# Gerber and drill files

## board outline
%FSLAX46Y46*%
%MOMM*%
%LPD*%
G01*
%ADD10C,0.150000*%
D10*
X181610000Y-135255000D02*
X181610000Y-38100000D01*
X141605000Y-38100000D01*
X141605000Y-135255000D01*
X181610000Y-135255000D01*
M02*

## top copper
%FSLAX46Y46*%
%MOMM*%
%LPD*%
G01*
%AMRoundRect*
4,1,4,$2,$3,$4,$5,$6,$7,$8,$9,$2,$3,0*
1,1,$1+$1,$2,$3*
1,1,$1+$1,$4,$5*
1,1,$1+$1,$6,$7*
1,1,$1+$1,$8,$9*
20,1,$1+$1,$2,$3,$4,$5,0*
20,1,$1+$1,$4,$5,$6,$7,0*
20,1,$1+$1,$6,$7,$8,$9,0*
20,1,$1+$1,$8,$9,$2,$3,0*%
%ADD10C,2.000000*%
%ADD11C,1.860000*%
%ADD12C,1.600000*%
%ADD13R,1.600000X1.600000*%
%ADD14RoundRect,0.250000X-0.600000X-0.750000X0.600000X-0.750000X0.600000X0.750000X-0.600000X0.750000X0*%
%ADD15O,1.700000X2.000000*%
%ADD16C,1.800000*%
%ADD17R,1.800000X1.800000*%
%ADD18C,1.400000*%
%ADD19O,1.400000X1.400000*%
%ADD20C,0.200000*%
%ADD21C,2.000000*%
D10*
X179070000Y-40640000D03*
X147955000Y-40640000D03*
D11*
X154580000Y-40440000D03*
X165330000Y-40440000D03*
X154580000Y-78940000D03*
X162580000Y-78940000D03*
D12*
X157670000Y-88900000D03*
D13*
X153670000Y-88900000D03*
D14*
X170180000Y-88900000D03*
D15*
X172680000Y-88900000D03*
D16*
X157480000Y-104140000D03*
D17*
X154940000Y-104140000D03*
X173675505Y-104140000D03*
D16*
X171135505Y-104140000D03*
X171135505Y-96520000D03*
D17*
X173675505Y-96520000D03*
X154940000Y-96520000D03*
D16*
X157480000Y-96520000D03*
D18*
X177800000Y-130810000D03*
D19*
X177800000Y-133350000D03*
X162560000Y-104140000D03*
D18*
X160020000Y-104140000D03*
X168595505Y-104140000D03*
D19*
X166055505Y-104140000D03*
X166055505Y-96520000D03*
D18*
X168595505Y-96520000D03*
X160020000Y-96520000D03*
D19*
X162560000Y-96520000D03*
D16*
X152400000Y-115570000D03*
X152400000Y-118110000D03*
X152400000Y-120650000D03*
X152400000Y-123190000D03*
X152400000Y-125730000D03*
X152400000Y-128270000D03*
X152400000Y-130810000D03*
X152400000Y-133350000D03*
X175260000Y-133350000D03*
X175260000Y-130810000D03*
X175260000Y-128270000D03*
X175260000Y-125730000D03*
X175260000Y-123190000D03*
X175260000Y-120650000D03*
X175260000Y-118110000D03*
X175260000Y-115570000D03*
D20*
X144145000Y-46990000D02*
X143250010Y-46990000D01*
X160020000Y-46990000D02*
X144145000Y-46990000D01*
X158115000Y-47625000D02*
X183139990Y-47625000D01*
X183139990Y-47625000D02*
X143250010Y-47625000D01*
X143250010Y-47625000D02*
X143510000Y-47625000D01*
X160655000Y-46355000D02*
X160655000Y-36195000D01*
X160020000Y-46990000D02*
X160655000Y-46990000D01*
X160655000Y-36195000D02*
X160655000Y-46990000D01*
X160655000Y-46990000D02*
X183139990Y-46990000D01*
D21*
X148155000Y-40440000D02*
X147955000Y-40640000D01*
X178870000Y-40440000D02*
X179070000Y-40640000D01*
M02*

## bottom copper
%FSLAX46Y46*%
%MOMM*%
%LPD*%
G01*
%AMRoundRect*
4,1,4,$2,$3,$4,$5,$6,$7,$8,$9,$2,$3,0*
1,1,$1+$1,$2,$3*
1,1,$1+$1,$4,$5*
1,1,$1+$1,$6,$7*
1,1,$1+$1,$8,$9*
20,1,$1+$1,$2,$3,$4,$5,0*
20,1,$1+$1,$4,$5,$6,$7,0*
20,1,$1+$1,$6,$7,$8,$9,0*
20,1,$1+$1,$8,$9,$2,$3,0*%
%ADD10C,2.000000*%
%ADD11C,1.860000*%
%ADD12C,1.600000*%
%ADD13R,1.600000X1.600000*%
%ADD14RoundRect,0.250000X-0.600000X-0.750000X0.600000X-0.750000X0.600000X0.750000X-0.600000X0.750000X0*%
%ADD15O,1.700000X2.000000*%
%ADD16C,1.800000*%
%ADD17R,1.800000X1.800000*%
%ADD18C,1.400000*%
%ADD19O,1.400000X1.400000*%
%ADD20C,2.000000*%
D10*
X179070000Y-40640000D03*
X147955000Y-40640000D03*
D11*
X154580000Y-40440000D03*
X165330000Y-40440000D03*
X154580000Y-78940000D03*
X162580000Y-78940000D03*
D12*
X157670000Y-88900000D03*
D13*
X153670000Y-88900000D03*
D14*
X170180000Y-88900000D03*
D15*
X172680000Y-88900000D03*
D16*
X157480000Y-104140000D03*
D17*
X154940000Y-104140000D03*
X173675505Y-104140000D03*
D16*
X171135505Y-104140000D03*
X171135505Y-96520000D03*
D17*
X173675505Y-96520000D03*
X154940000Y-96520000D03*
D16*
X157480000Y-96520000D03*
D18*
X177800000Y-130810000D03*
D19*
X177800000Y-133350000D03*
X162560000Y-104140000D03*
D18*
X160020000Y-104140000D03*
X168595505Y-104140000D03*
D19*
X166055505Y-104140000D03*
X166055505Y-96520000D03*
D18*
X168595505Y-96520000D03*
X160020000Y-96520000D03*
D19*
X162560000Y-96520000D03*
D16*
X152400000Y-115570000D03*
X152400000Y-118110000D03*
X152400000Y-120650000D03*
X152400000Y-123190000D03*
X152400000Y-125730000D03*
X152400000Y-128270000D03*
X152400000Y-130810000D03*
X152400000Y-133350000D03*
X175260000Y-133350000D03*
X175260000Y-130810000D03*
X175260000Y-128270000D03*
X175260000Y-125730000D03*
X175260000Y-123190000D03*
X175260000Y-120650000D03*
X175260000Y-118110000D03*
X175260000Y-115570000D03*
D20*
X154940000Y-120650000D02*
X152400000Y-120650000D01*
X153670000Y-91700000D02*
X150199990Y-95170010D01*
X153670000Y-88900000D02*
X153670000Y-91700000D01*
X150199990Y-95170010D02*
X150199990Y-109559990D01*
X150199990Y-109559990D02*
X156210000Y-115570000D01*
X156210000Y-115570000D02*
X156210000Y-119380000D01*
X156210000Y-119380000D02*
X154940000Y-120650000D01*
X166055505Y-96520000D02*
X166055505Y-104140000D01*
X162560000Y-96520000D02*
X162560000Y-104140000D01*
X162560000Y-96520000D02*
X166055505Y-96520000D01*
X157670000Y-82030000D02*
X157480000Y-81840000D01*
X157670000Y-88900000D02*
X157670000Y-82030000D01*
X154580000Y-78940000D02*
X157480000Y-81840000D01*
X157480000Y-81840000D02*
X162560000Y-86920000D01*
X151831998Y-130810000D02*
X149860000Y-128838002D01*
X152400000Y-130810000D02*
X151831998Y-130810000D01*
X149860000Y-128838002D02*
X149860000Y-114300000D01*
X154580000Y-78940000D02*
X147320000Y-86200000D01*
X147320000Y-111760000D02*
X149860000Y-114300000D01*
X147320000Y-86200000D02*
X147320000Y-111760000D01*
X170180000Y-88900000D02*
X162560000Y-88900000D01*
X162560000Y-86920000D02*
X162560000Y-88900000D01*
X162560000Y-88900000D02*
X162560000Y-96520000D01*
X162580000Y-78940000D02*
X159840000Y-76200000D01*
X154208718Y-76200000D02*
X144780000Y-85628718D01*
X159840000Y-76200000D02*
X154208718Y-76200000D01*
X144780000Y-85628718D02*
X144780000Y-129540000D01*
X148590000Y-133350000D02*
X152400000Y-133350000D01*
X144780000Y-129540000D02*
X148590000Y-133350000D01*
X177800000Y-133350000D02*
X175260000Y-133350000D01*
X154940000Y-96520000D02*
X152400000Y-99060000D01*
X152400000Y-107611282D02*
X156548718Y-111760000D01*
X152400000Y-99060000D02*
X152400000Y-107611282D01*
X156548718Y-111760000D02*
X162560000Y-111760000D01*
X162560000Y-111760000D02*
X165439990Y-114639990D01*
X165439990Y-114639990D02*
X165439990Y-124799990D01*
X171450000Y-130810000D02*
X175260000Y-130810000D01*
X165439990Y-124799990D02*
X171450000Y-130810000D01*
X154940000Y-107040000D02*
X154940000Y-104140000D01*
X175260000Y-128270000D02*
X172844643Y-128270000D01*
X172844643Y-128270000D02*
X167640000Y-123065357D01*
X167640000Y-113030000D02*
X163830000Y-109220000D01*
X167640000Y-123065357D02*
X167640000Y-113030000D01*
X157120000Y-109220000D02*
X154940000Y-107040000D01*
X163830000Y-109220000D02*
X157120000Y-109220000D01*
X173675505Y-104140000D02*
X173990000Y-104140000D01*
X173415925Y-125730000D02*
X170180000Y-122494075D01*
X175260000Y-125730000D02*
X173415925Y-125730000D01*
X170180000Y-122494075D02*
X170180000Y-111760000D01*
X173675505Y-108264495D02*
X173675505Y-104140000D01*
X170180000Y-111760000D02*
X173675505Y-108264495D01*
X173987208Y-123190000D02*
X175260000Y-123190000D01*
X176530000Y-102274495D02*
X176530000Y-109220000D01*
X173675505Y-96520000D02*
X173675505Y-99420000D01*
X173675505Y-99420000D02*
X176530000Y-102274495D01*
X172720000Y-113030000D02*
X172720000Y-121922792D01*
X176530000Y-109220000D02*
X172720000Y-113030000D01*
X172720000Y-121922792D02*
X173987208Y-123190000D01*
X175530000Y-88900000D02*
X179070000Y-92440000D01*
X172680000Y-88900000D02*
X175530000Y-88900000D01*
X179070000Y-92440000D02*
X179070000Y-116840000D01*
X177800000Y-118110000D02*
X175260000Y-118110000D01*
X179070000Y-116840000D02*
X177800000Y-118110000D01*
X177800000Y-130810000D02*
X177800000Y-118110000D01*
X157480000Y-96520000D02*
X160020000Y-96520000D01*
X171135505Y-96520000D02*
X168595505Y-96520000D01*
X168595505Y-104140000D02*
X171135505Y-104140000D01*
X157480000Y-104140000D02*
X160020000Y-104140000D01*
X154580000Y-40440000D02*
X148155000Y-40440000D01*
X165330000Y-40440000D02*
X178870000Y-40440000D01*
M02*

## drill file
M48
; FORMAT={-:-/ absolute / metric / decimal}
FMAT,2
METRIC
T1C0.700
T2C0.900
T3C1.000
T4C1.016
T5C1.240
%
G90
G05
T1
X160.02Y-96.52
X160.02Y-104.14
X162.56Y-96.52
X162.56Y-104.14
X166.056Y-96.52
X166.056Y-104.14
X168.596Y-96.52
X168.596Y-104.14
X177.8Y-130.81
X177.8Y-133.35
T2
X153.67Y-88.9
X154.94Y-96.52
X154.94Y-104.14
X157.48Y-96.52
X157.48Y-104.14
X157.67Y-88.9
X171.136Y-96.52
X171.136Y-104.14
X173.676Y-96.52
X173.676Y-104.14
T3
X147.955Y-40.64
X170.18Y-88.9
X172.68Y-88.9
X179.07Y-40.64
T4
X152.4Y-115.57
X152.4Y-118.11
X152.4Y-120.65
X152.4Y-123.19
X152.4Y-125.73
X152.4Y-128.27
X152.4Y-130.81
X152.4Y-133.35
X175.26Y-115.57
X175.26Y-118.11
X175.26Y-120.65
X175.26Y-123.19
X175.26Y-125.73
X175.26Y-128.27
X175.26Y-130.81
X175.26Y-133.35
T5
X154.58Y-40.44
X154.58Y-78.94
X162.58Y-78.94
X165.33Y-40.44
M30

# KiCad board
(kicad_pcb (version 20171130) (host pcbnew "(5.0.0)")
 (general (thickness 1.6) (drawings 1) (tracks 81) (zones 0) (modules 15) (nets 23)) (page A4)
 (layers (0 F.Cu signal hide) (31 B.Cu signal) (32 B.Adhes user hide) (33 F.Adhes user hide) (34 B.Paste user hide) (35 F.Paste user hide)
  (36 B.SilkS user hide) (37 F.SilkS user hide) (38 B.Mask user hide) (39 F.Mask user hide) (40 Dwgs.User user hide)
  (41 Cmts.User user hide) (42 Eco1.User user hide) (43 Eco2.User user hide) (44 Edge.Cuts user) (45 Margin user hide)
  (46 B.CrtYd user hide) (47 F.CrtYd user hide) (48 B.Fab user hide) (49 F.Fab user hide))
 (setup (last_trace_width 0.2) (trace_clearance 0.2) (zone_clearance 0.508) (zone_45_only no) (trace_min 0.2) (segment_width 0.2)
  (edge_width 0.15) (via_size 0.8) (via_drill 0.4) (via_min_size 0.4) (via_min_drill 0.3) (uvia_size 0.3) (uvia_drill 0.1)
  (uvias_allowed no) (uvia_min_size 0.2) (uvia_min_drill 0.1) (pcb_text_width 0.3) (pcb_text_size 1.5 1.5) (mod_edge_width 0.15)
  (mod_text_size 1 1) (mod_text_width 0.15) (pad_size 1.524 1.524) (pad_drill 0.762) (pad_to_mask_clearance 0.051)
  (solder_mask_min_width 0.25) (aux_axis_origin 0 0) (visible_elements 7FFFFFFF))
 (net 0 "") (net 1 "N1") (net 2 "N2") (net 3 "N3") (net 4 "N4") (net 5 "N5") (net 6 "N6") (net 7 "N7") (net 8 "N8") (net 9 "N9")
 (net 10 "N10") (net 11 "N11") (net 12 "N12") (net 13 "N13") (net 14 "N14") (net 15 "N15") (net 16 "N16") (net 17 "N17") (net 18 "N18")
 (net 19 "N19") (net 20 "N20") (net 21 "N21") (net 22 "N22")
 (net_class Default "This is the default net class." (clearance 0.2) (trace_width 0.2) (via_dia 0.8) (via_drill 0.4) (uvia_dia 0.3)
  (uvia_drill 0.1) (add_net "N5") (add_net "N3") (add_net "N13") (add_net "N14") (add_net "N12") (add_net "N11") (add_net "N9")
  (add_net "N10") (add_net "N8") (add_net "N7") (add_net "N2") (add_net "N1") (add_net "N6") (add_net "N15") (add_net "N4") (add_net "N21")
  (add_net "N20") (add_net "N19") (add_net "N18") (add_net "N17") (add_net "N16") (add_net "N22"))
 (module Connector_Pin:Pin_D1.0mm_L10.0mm (layer F.Cu) (at 179.07 40.64)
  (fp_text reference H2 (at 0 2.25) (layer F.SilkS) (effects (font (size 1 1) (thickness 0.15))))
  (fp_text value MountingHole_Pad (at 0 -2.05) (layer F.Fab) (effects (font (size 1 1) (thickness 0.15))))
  (pad 1 thru_hole circle (at 0 0) (size 2 2) (drill 1) (layers *.Cu *.Mask) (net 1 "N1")))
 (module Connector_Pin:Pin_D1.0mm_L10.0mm (layer F.Cu) (at 147.955 40.64)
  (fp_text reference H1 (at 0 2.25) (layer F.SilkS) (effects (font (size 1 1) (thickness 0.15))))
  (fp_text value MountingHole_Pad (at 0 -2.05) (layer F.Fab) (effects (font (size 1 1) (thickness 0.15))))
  (pad 1 thru_hole circle (at 0 0) (size 2 2) (drill 1) (layers *.Cu *.Mask) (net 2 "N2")))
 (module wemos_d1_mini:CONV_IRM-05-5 (layer F.Cu) (at 163.83 59.69 270)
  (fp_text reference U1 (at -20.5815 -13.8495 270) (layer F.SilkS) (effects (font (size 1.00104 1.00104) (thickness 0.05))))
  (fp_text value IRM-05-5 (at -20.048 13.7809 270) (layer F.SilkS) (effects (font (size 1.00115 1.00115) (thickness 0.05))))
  (pad AC/L thru_hole circle (at -19.25 9.25 270) (size 1.86 1.86) (drill 1.24) (layers *.Cu *.Mask) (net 2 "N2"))
  (pad AC/N thru_hole circle (at -19.25 -1.5 270) (size 1.86 1.86) (drill 1.24) (layers *.Cu *.Mask) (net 1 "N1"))
  (pad VNEG thru_hole circle (at 19.25 9.25 270) (size 1.86 1.86) (drill 1.24) (layers *.Cu *.Mask) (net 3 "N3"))
  (pad VPOS thru_hole circle (at 19.25 1.25 270) (size 1.86 1.86) (drill 1.24) (layers *.Cu *.Mask) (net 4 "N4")))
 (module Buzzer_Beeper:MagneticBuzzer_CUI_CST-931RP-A (layer F.Cu) (at 153.67 88.9 90)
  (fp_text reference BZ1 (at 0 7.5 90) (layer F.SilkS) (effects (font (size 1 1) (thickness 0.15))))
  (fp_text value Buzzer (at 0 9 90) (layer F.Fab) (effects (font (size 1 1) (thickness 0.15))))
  (pad 2 thru_hole circle (at 0 4 90) (size 1.6 1.6) (drill 0.9) (layers *.Cu *.Mask) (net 3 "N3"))
  (pad 1 thru_hole rect (at 0 0 90) (size 1.6 1.6) (drill 0.9) (layers *.Cu *.Mask) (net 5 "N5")))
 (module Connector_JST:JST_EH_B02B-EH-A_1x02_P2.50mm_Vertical (layer B.Cu) (at 170.18 88.9)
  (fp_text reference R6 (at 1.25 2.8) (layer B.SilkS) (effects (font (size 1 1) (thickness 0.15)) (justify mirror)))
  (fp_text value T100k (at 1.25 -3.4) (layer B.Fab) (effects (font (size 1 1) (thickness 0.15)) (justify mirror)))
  (pad 1 thru_hole roundrect (at 0 0) (size 1.7 2) (drill 1) (layers *.Cu *.Mask) (roundrect_rratio 0.147059) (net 3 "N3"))
  (pad 2 thru_hole oval (at 2.5 0) (size 1.7 2) (drill 1) (layers *.Cu *.Mask) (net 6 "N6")))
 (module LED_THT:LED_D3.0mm (layer F.Cu) (at 154.94 104.14)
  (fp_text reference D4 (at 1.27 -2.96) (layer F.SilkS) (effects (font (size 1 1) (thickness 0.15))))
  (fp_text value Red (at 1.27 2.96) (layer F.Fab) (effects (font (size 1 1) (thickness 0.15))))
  (pad 2 thru_hole circle (at 2.54 0) (size 1.8 1.8) (drill 0.9) (layers *.Cu *.Mask) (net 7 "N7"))
  (pad 1 thru_hole rect (at 0 0) (size 1.8 1.8) (drill 0.9) (layers *.Cu *.Mask) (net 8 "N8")))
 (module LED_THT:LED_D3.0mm (layer F.Cu) (at 173.675505 104.14 180)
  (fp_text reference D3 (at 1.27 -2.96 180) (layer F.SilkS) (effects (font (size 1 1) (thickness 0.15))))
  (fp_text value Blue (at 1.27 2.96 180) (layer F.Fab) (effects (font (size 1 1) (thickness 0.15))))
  (pad 1 thru_hole rect (at 0 0 180) (size 1.8 1.8) (drill 0.9) (layers *.Cu *.Mask) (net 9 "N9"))
  (pad 2 thru_hole circle (at 2.54 0 180) (size 1.8 1.8) (drill 0.9) (layers *.Cu *.Mask) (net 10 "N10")))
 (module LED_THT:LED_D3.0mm (layer F.Cu) (at 173.675505 96.52 180)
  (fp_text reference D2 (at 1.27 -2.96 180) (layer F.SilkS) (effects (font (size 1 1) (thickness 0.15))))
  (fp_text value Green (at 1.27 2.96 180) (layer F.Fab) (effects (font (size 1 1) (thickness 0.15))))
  (pad 2 thru_hole circle (at 2.54 0 180) (size 1.8 1.8) (drill 0.9) (layers *.Cu *.Mask) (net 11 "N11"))
  (pad 1 thru_hole rect (at 0 0 180) (size 1.8 1.8) (drill 0.9) (layers *.Cu *.Mask) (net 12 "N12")))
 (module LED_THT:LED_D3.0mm (layer F.Cu) (at 154.94 96.52)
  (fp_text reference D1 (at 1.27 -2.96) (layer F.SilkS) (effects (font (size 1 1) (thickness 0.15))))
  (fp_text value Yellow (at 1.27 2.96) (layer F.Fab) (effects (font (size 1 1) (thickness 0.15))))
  (pad 1 thru_hole rect (at 0 0) (size 1.8 1.8) (drill 0.9) (layers *.Cu *.Mask) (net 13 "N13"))
  (pad 2 thru_hole circle (at 2.54 0) (size 1.8 1.8) (drill 0.9) (layers *.Cu *.Mask) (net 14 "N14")))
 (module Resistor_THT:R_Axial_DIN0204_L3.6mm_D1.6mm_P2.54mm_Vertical (layer F.Cu) (at 177.8 130.81 270)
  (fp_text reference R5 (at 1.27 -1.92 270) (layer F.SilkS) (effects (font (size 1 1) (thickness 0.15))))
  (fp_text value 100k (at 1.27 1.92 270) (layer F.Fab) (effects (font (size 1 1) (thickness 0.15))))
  (pad 1 thru_hole circle (at 0 0 270) (size 1.4 1.4) (drill 0.7) (layers *.Cu *.Mask) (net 6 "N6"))
  (pad 2 thru_hole oval (at 2.54 0 270) (size 1.4 1.4) (drill 0.7) (layers *.Cu *.Mask) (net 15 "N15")))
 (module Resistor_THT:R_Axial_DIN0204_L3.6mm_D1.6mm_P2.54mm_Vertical (layer F.Cu) (at 160.02 104.14)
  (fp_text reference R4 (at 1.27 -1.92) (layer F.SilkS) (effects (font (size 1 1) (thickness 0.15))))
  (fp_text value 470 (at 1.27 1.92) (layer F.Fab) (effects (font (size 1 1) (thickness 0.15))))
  (pad 2 thru_hole oval (at 2.54 0) (size 1.4 1.4) (drill 0.7) (layers *.Cu *.Mask) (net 3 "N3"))
  (pad 1 thru_hole circle (at 0 0) (size 1.4 1.4) (drill 0.7) (layers *.Cu *.Mask) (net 7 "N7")))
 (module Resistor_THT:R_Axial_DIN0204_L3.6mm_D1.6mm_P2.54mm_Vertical (layer F.Cu) (at 168.595505 104.14 180)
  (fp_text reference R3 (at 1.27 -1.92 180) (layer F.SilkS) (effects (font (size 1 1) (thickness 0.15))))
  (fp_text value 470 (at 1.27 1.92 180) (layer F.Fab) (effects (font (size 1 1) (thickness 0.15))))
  (pad 1 thru_hole circle (at 0 0 180) (size 1.4 1.4) (drill 0.7) (layers *.Cu *.Mask) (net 10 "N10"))
  (pad 2 thru_hole oval (at 2.54 0 180) (size 1.4 1.4) (drill 0.7) (layers *.Cu *.Mask) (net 3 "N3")))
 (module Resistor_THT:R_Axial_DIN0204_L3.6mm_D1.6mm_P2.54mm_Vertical (layer F.Cu) (at 168.595505 96.52 180)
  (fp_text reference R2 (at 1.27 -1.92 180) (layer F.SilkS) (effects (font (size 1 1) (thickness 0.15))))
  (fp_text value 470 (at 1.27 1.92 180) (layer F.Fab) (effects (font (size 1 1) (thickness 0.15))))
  (pad 2 thru_hole oval (at 2.54 0 180) (size 1.4 1.4) (drill 0.7) (layers *.Cu *.Mask) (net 3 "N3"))
  (pad 1 thru_hole circle (at 0 0 180) (size 1.4 1.4) (drill 0.7) (layers *.Cu *.Mask) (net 11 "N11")))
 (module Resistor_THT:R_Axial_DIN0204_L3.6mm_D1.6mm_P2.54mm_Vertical (layer F.Cu) (at 160.02 96.52)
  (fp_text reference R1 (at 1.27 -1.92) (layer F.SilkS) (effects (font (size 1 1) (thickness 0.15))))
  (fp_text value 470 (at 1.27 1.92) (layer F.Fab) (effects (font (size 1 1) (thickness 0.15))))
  (pad 1 thru_hole circle (at 0 0) (size 1.4 1.4) (drill 0.7) (layers *.Cu *.Mask) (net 14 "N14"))
  (pad 2 thru_hole oval (at 2.54 0) (size 1.4 1.4) (drill 0.7) (layers *.Cu *.Mask) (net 3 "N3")))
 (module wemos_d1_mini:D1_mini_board (layer F.Cu) (at 163.83 125.73)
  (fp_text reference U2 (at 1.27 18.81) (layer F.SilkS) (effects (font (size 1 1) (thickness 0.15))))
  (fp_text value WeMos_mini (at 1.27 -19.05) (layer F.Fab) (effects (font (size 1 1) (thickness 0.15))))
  (pad 8 thru_hole circle (at -11.43 -10.16) (size 1.8 1.8) (drill 1.016) (layers *.Cu *.Mask F.SilkS) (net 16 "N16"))
  (pad 7 thru_hole circle (at -11.43 -7.62) (size 1.8 1.8) (drill 1.016) (layers *.Cu *.Mask F.SilkS) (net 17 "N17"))
  (pad 6 thru_hole circle (at -11.43 -5.08) (size 1.8 1.8) (drill 1.016) (layers *.Cu *.Mask F.SilkS) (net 5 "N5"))
  (pad 5 thru_hole circle (at -11.43 -2.54) (size 1.8 1.8) (drill 1.016) (layers *.Cu *.Mask F.SilkS) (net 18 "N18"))
  (pad 4 thru_hole circle (at -11.43 0) (size 1.8 1.8) (drill 1.016) (layers *.Cu *.Mask F.SilkS) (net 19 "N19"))
  (pad 3 thru_hole circle (at -11.43 2.54) (size 1.8 1.8) (drill 1.016) (layers *.Cu *.Mask F.SilkS) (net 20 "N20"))
  (pad 2 thru_hole circle (at -11.43 5.08) (size 1.8 1.8) (drill 1.016) (layers *.Cu *.Mask F.SilkS) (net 3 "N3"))
  (pad 1 thru_hole circle (at -11.43 7.62) (size 1.8 1.8) (drill 1.016) (layers *.Cu *.Mask F.SilkS) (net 4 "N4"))
  (pad 16 thru_hole circle (at 11.43 7.62) (size 1.8 1.8) (drill 1.016) (layers *.Cu *.Mask F.SilkS) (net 15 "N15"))
  (pad 15 thru_hole circle (at 11.43 5.08) (size 1.8 1.8) (drill 1.016) (layers *.Cu *.Mask F.SilkS) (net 13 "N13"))
  (pad 14 thru_hole circle (at 11.43 2.54) (size 1.8 1.8) (drill 1.016) (layers *.Cu *.Mask F.SilkS) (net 8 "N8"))
  (pad 13 thru_hole circle (at 11.43 0) (size 1.8 1.8) (drill 1.016) (layers *.Cu *.Mask F.SilkS) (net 9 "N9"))
  (pad 12 thru_hole circle (at 11.43 -2.54) (size 1.8 1.8) (drill 1.016) (layers *.Cu *.Mask F.SilkS) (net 12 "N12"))
  (pad 11 thru_hole circle (at 11.43 -5.08) (size 1.8 1.8) (drill 1.016) (layers *.Cu *.Mask F.SilkS) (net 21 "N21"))
  (pad 10 thru_hole circle (at 11.43 -7.62) (size 1.8 1.8) (drill 1.016) (layers *.Cu *.Mask F.SilkS) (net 6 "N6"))
  (pad 9 thru_hole circle (at 11.43 -10.16) (size 1.8 1.8) (drill 1.016) (layers *.Cu *.Mask F.SilkS) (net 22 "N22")))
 (gr_poly (pts (xy 181.61 135.255) (xy 181.61 38.1) (xy 141.605 38.1) (xy 141.605 135.255)) (layer Edge.Cuts) (width 0.15))
 (segment (start 144.145 46.99) (end 143.25001 46.99) (width 0.2) (layer F.Cu) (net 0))
 (segment (start 160.02 46.99) (end 144.145 46.99) (width 0.2) (layer F.Cu) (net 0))
 (segment (start 158.115 47.625) (end 183.13999 47.625) (width 0.2) (layer F.Cu) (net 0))
 (segment (start 183.13999 47.625) (end 143.25001 47.625) (width 0.2) (layer F.Cu) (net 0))
 (segment (start 143.25001 47.625) (end 143.51 47.625) (width 0.2) (layer F.Cu) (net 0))
 (segment (start 160.655 46.355) (end 160.655 36.195) (width 0.2) (layer F.Cu) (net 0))
 (segment (start 160.02 46.99) (end 160.655 46.99) (width 0.2) (layer F.Cu) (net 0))
 (segment (start 160.655 36.195) (end 160.655 46.99) (width 0.2) (layer F.Cu) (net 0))
 (segment (start 160.655 46.99) (end 183.13999 46.99) (width 0.2) (layer F.Cu) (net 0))
 (segment (start 154.94 120.65) (end 152.4 120.65) (width 2) (layer B.Cu) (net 5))
 (segment (start 153.67 91.7) (end 150.19999 95.17001) (width 2) (layer B.Cu) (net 5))
 (segment (start 153.67 88.9) (end 153.67 91.7) (width 2) (layer B.Cu) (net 5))
 (segment (start 150.19999 95.17001) (end 150.19999 109.55999) (width 2) (layer B.Cu) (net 5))
 (segment (start 150.19999 109.55999) (end 156.21 115.57) (width 2) (layer B.Cu) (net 5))
 (segment (start 156.21 115.57) (end 156.21 119.38) (width 2) (layer B.Cu) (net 5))
 (segment (start 156.21 119.38) (end 154.94 120.65) (width 2) (layer B.Cu) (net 5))
 (segment (start 166.055505 96.52) (end 166.055505 104.14) (width 2) (layer B.Cu) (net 3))
 (segment (start 162.56 96.52) (end 162.56 104.14) (width 2) (layer B.Cu) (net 3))
 (segment (start 162.56 96.52) (end 166.055505 96.52) (width 2) (layer B.Cu) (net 3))
 (segment (start 157.67 82.03) (end 157.48 81.84) (width 2) (layer B.Cu) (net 3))
 (segment (start 157.67 88.9) (end 157.67 82.03) (width 2) (layer B.Cu) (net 3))
 (segment (start 154.58 78.94) (end 157.48 81.84) (width 2) (layer B.Cu) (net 3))
 (segment (start 157.48 81.84) (end 162.56 86.92) (width 2) (layer B.Cu) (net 3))
 (segment (start 151.831998 130.81) (end 149.86 128.838002) (width 2) (layer B.Cu) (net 3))
 (segment (start 152.4 130.81) (end 151.831998 130.81) (width 2) (layer B.Cu) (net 3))
 (segment (start 149.86 128.838002) (end 149.86 114.3) (width 2) (layer B.Cu) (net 3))
 (segment (start 154.58 78.94) (end 147.32 86.2) (width 2) (layer B.Cu) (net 3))
 (segment (start 147.32 111.76) (end 149.86 114.3) (width 2) (layer B.Cu) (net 3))
 (segment (start 147.32 86.2) (end 147.32 111.76) (width 2) (layer B.Cu) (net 3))
 (segment (start 170.18 88.9) (end 162.56 88.9) (width 2) (layer B.Cu) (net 3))
 (segment (start 162.56 86.92) (end 162.56 88.9) (width 2) (layer B.Cu) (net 3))
 (segment (start 162.56 88.9) (end 162.56 96.52) (width 2) (layer B.Cu) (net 3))
 (segment (start 162.58 78.94) (end 159.84 76.2) (width 2) (layer B.Cu) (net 4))
 (segment (start 154.208718 76.2) (end 144.78 85.628718) (width 2) (layer B.Cu) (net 4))
 (segment (start 159.84 76.2) (end 154.208718 76.2) (width 2) (layer B.Cu) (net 4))
 (segment (start 144.78 85.628718) (end 144.78 129.54) (width 2) (layer B.Cu) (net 4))
 (segment (start 148.59 133.35) (end 152.4 133.35) (width 2) (layer B.Cu) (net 4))
 (segment (start 144.78 129.54) (end 148.59 133.35) (width 2) (layer B.Cu) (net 4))
 (segment (start 177.8 133.35) (end 175.26 133.35) (width 2) (layer B.Cu) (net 15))
 (segment (start 154.94 96.52) (end 152.4 99.06) (width 2) (layer B.Cu) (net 13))
 (segment (start 152.4 107.611282) (end 156.548718 111.76) (width 2) (layer B.Cu) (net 13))
 (segment (start 152.4 99.06) (end 152.4 107.611282) (width 2) (layer B.Cu) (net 13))
 (segment (start 156.548718 111.76) (end 162.56 111.76) (width 2) (layer B.Cu) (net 13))
 (segment (start 162.56 111.76) (end 165.43999 114.63999) (width 2) (layer B.Cu) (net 13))
 (segment (start 165.43999 114.63999) (end 165.43999 124.79999) (width 2) (layer B.Cu) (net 13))
 (segment (start 171.45 130.81) (end 175.26 130.81) (width 2) (layer B.Cu) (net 13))
 (segment (start 165.43999 124.79999) (end 171.45 130.81) (width 2) (layer B.Cu) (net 13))
 (segment (start 154.94 107.04) (end 154.94 104.14) (width 2) (layer B.Cu) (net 8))
 (segment (start 175.26 128.27) (end 172.844643 128.27) (width 2) (layer B.Cu) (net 8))
 (segment (start 172.844643 128.27) (end 167.64 123.065357) (width 2) (layer B.Cu) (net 8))
 (segment (start 167.64 113.03) (end 163.83 109.22) (width 2) (layer B.Cu) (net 8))
 (segment (start 167.64 123.065357) (end 167.64 113.03) (width 2) (layer B.Cu) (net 8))
 (segment (start 157.12 109.22) (end 154.94 107.04) (width 2) (layer B.Cu) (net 8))
 (segment (start 163.83 109.22) (end 157.12 109.22) (width 2) (layer B.Cu) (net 8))
 (segment (start 173.675505 104.14) (end 173.99 104.14) (width 2) (layer B.Cu) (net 9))
 (segment (start 173.415925 125.73) (end 170.18 122.494075) (width 2) (layer B.Cu) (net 9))
 (segment (start 175.26 125.73) (end 173.415925 125.73) (width 2) (layer B.Cu) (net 9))
 (segment (start 170.18 122.494075) (end 170.18 111.76) (width 2) (layer B.Cu) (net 9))
 (segment (start 173.675505 108.264495) (end 173.675505 104.14) (width 2) (layer B.Cu) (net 9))
 (segment (start 170.18 111.76) (end 173.675505 108.264495) (width 2) (layer B.Cu) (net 9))
 (segment (start 173.987208 123.19) (end 175.26 123.19) (width 2) (layer B.Cu) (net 12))
 (segment (start 176.53 102.274495) (end 176.53 109.22) (width 2) (layer B.Cu) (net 12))
 (segment (start 173.675505 96.52) (end 173.675505 99.42) (width 2) (layer B.Cu) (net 12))
 (segment (start 173.675505 99.42) (end 176.53 102.274495) (width 2) (layer B.Cu) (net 12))
 (segment (start 172.72 113.03) (end 172.72 121.922792) (width 2) (layer B.Cu) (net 12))
 (segment (start 176.53 109.22) (end 172.72 113.03) (width 2) (layer B.Cu) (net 12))
 (segment (start 172.72 121.922792) (end 173.987208 123.19) (width 2) (layer B.Cu) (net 12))
 (segment (start 175.53 88.9) (end 179.07 92.44) (width 2) (layer B.Cu) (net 6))
 (segment (start 172.68 88.9) (end 175.53 88.9) (width 2) (layer B.Cu) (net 6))
 (segment (start 179.07 92.44) (end 179.07 116.84) (width 2) (layer B.Cu) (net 6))
 (segment (start 177.8 118.11) (end 175.26 118.11) (width 2) (layer B.Cu) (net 6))
 (segment (start 179.07 116.84) (end 177.8 118.11) (width 2) (layer B.Cu) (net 6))
 (segment (start 177.8 130.81) (end 177.8 118.11) (width 2) (layer B.Cu) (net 6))
 (segment (start 157.48 96.52) (end 160.02 96.52) (width 2) (layer B.Cu) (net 14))
 (segment (start 171.135505 96.52) (end 168.595505 96.52) (width 2) (layer B.Cu) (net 11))
 (segment (start 168.595505 104.14) (end 171.135505 104.14) (width 2) (layer B.Cu) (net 10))
 (segment (start 157.48 104.14) (end 160.02 104.14) (width 2) (layer B.Cu) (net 7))
 (segment (start 148.155 40.44) (end 147.955 40.64) (width 2) (layer F.Cu) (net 2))
 (segment (start 154.58 40.44) (end 148.155 40.44) (width 2) (layer B.Cu) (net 2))
 (segment (start 178.87 40.44) (end 179.07 40.64) (width 2) (layer F.Cu) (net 1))
 (segment (start 165.33 40.44) (end 178.87 40.44) (width 2) (layer B.Cu) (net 1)))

